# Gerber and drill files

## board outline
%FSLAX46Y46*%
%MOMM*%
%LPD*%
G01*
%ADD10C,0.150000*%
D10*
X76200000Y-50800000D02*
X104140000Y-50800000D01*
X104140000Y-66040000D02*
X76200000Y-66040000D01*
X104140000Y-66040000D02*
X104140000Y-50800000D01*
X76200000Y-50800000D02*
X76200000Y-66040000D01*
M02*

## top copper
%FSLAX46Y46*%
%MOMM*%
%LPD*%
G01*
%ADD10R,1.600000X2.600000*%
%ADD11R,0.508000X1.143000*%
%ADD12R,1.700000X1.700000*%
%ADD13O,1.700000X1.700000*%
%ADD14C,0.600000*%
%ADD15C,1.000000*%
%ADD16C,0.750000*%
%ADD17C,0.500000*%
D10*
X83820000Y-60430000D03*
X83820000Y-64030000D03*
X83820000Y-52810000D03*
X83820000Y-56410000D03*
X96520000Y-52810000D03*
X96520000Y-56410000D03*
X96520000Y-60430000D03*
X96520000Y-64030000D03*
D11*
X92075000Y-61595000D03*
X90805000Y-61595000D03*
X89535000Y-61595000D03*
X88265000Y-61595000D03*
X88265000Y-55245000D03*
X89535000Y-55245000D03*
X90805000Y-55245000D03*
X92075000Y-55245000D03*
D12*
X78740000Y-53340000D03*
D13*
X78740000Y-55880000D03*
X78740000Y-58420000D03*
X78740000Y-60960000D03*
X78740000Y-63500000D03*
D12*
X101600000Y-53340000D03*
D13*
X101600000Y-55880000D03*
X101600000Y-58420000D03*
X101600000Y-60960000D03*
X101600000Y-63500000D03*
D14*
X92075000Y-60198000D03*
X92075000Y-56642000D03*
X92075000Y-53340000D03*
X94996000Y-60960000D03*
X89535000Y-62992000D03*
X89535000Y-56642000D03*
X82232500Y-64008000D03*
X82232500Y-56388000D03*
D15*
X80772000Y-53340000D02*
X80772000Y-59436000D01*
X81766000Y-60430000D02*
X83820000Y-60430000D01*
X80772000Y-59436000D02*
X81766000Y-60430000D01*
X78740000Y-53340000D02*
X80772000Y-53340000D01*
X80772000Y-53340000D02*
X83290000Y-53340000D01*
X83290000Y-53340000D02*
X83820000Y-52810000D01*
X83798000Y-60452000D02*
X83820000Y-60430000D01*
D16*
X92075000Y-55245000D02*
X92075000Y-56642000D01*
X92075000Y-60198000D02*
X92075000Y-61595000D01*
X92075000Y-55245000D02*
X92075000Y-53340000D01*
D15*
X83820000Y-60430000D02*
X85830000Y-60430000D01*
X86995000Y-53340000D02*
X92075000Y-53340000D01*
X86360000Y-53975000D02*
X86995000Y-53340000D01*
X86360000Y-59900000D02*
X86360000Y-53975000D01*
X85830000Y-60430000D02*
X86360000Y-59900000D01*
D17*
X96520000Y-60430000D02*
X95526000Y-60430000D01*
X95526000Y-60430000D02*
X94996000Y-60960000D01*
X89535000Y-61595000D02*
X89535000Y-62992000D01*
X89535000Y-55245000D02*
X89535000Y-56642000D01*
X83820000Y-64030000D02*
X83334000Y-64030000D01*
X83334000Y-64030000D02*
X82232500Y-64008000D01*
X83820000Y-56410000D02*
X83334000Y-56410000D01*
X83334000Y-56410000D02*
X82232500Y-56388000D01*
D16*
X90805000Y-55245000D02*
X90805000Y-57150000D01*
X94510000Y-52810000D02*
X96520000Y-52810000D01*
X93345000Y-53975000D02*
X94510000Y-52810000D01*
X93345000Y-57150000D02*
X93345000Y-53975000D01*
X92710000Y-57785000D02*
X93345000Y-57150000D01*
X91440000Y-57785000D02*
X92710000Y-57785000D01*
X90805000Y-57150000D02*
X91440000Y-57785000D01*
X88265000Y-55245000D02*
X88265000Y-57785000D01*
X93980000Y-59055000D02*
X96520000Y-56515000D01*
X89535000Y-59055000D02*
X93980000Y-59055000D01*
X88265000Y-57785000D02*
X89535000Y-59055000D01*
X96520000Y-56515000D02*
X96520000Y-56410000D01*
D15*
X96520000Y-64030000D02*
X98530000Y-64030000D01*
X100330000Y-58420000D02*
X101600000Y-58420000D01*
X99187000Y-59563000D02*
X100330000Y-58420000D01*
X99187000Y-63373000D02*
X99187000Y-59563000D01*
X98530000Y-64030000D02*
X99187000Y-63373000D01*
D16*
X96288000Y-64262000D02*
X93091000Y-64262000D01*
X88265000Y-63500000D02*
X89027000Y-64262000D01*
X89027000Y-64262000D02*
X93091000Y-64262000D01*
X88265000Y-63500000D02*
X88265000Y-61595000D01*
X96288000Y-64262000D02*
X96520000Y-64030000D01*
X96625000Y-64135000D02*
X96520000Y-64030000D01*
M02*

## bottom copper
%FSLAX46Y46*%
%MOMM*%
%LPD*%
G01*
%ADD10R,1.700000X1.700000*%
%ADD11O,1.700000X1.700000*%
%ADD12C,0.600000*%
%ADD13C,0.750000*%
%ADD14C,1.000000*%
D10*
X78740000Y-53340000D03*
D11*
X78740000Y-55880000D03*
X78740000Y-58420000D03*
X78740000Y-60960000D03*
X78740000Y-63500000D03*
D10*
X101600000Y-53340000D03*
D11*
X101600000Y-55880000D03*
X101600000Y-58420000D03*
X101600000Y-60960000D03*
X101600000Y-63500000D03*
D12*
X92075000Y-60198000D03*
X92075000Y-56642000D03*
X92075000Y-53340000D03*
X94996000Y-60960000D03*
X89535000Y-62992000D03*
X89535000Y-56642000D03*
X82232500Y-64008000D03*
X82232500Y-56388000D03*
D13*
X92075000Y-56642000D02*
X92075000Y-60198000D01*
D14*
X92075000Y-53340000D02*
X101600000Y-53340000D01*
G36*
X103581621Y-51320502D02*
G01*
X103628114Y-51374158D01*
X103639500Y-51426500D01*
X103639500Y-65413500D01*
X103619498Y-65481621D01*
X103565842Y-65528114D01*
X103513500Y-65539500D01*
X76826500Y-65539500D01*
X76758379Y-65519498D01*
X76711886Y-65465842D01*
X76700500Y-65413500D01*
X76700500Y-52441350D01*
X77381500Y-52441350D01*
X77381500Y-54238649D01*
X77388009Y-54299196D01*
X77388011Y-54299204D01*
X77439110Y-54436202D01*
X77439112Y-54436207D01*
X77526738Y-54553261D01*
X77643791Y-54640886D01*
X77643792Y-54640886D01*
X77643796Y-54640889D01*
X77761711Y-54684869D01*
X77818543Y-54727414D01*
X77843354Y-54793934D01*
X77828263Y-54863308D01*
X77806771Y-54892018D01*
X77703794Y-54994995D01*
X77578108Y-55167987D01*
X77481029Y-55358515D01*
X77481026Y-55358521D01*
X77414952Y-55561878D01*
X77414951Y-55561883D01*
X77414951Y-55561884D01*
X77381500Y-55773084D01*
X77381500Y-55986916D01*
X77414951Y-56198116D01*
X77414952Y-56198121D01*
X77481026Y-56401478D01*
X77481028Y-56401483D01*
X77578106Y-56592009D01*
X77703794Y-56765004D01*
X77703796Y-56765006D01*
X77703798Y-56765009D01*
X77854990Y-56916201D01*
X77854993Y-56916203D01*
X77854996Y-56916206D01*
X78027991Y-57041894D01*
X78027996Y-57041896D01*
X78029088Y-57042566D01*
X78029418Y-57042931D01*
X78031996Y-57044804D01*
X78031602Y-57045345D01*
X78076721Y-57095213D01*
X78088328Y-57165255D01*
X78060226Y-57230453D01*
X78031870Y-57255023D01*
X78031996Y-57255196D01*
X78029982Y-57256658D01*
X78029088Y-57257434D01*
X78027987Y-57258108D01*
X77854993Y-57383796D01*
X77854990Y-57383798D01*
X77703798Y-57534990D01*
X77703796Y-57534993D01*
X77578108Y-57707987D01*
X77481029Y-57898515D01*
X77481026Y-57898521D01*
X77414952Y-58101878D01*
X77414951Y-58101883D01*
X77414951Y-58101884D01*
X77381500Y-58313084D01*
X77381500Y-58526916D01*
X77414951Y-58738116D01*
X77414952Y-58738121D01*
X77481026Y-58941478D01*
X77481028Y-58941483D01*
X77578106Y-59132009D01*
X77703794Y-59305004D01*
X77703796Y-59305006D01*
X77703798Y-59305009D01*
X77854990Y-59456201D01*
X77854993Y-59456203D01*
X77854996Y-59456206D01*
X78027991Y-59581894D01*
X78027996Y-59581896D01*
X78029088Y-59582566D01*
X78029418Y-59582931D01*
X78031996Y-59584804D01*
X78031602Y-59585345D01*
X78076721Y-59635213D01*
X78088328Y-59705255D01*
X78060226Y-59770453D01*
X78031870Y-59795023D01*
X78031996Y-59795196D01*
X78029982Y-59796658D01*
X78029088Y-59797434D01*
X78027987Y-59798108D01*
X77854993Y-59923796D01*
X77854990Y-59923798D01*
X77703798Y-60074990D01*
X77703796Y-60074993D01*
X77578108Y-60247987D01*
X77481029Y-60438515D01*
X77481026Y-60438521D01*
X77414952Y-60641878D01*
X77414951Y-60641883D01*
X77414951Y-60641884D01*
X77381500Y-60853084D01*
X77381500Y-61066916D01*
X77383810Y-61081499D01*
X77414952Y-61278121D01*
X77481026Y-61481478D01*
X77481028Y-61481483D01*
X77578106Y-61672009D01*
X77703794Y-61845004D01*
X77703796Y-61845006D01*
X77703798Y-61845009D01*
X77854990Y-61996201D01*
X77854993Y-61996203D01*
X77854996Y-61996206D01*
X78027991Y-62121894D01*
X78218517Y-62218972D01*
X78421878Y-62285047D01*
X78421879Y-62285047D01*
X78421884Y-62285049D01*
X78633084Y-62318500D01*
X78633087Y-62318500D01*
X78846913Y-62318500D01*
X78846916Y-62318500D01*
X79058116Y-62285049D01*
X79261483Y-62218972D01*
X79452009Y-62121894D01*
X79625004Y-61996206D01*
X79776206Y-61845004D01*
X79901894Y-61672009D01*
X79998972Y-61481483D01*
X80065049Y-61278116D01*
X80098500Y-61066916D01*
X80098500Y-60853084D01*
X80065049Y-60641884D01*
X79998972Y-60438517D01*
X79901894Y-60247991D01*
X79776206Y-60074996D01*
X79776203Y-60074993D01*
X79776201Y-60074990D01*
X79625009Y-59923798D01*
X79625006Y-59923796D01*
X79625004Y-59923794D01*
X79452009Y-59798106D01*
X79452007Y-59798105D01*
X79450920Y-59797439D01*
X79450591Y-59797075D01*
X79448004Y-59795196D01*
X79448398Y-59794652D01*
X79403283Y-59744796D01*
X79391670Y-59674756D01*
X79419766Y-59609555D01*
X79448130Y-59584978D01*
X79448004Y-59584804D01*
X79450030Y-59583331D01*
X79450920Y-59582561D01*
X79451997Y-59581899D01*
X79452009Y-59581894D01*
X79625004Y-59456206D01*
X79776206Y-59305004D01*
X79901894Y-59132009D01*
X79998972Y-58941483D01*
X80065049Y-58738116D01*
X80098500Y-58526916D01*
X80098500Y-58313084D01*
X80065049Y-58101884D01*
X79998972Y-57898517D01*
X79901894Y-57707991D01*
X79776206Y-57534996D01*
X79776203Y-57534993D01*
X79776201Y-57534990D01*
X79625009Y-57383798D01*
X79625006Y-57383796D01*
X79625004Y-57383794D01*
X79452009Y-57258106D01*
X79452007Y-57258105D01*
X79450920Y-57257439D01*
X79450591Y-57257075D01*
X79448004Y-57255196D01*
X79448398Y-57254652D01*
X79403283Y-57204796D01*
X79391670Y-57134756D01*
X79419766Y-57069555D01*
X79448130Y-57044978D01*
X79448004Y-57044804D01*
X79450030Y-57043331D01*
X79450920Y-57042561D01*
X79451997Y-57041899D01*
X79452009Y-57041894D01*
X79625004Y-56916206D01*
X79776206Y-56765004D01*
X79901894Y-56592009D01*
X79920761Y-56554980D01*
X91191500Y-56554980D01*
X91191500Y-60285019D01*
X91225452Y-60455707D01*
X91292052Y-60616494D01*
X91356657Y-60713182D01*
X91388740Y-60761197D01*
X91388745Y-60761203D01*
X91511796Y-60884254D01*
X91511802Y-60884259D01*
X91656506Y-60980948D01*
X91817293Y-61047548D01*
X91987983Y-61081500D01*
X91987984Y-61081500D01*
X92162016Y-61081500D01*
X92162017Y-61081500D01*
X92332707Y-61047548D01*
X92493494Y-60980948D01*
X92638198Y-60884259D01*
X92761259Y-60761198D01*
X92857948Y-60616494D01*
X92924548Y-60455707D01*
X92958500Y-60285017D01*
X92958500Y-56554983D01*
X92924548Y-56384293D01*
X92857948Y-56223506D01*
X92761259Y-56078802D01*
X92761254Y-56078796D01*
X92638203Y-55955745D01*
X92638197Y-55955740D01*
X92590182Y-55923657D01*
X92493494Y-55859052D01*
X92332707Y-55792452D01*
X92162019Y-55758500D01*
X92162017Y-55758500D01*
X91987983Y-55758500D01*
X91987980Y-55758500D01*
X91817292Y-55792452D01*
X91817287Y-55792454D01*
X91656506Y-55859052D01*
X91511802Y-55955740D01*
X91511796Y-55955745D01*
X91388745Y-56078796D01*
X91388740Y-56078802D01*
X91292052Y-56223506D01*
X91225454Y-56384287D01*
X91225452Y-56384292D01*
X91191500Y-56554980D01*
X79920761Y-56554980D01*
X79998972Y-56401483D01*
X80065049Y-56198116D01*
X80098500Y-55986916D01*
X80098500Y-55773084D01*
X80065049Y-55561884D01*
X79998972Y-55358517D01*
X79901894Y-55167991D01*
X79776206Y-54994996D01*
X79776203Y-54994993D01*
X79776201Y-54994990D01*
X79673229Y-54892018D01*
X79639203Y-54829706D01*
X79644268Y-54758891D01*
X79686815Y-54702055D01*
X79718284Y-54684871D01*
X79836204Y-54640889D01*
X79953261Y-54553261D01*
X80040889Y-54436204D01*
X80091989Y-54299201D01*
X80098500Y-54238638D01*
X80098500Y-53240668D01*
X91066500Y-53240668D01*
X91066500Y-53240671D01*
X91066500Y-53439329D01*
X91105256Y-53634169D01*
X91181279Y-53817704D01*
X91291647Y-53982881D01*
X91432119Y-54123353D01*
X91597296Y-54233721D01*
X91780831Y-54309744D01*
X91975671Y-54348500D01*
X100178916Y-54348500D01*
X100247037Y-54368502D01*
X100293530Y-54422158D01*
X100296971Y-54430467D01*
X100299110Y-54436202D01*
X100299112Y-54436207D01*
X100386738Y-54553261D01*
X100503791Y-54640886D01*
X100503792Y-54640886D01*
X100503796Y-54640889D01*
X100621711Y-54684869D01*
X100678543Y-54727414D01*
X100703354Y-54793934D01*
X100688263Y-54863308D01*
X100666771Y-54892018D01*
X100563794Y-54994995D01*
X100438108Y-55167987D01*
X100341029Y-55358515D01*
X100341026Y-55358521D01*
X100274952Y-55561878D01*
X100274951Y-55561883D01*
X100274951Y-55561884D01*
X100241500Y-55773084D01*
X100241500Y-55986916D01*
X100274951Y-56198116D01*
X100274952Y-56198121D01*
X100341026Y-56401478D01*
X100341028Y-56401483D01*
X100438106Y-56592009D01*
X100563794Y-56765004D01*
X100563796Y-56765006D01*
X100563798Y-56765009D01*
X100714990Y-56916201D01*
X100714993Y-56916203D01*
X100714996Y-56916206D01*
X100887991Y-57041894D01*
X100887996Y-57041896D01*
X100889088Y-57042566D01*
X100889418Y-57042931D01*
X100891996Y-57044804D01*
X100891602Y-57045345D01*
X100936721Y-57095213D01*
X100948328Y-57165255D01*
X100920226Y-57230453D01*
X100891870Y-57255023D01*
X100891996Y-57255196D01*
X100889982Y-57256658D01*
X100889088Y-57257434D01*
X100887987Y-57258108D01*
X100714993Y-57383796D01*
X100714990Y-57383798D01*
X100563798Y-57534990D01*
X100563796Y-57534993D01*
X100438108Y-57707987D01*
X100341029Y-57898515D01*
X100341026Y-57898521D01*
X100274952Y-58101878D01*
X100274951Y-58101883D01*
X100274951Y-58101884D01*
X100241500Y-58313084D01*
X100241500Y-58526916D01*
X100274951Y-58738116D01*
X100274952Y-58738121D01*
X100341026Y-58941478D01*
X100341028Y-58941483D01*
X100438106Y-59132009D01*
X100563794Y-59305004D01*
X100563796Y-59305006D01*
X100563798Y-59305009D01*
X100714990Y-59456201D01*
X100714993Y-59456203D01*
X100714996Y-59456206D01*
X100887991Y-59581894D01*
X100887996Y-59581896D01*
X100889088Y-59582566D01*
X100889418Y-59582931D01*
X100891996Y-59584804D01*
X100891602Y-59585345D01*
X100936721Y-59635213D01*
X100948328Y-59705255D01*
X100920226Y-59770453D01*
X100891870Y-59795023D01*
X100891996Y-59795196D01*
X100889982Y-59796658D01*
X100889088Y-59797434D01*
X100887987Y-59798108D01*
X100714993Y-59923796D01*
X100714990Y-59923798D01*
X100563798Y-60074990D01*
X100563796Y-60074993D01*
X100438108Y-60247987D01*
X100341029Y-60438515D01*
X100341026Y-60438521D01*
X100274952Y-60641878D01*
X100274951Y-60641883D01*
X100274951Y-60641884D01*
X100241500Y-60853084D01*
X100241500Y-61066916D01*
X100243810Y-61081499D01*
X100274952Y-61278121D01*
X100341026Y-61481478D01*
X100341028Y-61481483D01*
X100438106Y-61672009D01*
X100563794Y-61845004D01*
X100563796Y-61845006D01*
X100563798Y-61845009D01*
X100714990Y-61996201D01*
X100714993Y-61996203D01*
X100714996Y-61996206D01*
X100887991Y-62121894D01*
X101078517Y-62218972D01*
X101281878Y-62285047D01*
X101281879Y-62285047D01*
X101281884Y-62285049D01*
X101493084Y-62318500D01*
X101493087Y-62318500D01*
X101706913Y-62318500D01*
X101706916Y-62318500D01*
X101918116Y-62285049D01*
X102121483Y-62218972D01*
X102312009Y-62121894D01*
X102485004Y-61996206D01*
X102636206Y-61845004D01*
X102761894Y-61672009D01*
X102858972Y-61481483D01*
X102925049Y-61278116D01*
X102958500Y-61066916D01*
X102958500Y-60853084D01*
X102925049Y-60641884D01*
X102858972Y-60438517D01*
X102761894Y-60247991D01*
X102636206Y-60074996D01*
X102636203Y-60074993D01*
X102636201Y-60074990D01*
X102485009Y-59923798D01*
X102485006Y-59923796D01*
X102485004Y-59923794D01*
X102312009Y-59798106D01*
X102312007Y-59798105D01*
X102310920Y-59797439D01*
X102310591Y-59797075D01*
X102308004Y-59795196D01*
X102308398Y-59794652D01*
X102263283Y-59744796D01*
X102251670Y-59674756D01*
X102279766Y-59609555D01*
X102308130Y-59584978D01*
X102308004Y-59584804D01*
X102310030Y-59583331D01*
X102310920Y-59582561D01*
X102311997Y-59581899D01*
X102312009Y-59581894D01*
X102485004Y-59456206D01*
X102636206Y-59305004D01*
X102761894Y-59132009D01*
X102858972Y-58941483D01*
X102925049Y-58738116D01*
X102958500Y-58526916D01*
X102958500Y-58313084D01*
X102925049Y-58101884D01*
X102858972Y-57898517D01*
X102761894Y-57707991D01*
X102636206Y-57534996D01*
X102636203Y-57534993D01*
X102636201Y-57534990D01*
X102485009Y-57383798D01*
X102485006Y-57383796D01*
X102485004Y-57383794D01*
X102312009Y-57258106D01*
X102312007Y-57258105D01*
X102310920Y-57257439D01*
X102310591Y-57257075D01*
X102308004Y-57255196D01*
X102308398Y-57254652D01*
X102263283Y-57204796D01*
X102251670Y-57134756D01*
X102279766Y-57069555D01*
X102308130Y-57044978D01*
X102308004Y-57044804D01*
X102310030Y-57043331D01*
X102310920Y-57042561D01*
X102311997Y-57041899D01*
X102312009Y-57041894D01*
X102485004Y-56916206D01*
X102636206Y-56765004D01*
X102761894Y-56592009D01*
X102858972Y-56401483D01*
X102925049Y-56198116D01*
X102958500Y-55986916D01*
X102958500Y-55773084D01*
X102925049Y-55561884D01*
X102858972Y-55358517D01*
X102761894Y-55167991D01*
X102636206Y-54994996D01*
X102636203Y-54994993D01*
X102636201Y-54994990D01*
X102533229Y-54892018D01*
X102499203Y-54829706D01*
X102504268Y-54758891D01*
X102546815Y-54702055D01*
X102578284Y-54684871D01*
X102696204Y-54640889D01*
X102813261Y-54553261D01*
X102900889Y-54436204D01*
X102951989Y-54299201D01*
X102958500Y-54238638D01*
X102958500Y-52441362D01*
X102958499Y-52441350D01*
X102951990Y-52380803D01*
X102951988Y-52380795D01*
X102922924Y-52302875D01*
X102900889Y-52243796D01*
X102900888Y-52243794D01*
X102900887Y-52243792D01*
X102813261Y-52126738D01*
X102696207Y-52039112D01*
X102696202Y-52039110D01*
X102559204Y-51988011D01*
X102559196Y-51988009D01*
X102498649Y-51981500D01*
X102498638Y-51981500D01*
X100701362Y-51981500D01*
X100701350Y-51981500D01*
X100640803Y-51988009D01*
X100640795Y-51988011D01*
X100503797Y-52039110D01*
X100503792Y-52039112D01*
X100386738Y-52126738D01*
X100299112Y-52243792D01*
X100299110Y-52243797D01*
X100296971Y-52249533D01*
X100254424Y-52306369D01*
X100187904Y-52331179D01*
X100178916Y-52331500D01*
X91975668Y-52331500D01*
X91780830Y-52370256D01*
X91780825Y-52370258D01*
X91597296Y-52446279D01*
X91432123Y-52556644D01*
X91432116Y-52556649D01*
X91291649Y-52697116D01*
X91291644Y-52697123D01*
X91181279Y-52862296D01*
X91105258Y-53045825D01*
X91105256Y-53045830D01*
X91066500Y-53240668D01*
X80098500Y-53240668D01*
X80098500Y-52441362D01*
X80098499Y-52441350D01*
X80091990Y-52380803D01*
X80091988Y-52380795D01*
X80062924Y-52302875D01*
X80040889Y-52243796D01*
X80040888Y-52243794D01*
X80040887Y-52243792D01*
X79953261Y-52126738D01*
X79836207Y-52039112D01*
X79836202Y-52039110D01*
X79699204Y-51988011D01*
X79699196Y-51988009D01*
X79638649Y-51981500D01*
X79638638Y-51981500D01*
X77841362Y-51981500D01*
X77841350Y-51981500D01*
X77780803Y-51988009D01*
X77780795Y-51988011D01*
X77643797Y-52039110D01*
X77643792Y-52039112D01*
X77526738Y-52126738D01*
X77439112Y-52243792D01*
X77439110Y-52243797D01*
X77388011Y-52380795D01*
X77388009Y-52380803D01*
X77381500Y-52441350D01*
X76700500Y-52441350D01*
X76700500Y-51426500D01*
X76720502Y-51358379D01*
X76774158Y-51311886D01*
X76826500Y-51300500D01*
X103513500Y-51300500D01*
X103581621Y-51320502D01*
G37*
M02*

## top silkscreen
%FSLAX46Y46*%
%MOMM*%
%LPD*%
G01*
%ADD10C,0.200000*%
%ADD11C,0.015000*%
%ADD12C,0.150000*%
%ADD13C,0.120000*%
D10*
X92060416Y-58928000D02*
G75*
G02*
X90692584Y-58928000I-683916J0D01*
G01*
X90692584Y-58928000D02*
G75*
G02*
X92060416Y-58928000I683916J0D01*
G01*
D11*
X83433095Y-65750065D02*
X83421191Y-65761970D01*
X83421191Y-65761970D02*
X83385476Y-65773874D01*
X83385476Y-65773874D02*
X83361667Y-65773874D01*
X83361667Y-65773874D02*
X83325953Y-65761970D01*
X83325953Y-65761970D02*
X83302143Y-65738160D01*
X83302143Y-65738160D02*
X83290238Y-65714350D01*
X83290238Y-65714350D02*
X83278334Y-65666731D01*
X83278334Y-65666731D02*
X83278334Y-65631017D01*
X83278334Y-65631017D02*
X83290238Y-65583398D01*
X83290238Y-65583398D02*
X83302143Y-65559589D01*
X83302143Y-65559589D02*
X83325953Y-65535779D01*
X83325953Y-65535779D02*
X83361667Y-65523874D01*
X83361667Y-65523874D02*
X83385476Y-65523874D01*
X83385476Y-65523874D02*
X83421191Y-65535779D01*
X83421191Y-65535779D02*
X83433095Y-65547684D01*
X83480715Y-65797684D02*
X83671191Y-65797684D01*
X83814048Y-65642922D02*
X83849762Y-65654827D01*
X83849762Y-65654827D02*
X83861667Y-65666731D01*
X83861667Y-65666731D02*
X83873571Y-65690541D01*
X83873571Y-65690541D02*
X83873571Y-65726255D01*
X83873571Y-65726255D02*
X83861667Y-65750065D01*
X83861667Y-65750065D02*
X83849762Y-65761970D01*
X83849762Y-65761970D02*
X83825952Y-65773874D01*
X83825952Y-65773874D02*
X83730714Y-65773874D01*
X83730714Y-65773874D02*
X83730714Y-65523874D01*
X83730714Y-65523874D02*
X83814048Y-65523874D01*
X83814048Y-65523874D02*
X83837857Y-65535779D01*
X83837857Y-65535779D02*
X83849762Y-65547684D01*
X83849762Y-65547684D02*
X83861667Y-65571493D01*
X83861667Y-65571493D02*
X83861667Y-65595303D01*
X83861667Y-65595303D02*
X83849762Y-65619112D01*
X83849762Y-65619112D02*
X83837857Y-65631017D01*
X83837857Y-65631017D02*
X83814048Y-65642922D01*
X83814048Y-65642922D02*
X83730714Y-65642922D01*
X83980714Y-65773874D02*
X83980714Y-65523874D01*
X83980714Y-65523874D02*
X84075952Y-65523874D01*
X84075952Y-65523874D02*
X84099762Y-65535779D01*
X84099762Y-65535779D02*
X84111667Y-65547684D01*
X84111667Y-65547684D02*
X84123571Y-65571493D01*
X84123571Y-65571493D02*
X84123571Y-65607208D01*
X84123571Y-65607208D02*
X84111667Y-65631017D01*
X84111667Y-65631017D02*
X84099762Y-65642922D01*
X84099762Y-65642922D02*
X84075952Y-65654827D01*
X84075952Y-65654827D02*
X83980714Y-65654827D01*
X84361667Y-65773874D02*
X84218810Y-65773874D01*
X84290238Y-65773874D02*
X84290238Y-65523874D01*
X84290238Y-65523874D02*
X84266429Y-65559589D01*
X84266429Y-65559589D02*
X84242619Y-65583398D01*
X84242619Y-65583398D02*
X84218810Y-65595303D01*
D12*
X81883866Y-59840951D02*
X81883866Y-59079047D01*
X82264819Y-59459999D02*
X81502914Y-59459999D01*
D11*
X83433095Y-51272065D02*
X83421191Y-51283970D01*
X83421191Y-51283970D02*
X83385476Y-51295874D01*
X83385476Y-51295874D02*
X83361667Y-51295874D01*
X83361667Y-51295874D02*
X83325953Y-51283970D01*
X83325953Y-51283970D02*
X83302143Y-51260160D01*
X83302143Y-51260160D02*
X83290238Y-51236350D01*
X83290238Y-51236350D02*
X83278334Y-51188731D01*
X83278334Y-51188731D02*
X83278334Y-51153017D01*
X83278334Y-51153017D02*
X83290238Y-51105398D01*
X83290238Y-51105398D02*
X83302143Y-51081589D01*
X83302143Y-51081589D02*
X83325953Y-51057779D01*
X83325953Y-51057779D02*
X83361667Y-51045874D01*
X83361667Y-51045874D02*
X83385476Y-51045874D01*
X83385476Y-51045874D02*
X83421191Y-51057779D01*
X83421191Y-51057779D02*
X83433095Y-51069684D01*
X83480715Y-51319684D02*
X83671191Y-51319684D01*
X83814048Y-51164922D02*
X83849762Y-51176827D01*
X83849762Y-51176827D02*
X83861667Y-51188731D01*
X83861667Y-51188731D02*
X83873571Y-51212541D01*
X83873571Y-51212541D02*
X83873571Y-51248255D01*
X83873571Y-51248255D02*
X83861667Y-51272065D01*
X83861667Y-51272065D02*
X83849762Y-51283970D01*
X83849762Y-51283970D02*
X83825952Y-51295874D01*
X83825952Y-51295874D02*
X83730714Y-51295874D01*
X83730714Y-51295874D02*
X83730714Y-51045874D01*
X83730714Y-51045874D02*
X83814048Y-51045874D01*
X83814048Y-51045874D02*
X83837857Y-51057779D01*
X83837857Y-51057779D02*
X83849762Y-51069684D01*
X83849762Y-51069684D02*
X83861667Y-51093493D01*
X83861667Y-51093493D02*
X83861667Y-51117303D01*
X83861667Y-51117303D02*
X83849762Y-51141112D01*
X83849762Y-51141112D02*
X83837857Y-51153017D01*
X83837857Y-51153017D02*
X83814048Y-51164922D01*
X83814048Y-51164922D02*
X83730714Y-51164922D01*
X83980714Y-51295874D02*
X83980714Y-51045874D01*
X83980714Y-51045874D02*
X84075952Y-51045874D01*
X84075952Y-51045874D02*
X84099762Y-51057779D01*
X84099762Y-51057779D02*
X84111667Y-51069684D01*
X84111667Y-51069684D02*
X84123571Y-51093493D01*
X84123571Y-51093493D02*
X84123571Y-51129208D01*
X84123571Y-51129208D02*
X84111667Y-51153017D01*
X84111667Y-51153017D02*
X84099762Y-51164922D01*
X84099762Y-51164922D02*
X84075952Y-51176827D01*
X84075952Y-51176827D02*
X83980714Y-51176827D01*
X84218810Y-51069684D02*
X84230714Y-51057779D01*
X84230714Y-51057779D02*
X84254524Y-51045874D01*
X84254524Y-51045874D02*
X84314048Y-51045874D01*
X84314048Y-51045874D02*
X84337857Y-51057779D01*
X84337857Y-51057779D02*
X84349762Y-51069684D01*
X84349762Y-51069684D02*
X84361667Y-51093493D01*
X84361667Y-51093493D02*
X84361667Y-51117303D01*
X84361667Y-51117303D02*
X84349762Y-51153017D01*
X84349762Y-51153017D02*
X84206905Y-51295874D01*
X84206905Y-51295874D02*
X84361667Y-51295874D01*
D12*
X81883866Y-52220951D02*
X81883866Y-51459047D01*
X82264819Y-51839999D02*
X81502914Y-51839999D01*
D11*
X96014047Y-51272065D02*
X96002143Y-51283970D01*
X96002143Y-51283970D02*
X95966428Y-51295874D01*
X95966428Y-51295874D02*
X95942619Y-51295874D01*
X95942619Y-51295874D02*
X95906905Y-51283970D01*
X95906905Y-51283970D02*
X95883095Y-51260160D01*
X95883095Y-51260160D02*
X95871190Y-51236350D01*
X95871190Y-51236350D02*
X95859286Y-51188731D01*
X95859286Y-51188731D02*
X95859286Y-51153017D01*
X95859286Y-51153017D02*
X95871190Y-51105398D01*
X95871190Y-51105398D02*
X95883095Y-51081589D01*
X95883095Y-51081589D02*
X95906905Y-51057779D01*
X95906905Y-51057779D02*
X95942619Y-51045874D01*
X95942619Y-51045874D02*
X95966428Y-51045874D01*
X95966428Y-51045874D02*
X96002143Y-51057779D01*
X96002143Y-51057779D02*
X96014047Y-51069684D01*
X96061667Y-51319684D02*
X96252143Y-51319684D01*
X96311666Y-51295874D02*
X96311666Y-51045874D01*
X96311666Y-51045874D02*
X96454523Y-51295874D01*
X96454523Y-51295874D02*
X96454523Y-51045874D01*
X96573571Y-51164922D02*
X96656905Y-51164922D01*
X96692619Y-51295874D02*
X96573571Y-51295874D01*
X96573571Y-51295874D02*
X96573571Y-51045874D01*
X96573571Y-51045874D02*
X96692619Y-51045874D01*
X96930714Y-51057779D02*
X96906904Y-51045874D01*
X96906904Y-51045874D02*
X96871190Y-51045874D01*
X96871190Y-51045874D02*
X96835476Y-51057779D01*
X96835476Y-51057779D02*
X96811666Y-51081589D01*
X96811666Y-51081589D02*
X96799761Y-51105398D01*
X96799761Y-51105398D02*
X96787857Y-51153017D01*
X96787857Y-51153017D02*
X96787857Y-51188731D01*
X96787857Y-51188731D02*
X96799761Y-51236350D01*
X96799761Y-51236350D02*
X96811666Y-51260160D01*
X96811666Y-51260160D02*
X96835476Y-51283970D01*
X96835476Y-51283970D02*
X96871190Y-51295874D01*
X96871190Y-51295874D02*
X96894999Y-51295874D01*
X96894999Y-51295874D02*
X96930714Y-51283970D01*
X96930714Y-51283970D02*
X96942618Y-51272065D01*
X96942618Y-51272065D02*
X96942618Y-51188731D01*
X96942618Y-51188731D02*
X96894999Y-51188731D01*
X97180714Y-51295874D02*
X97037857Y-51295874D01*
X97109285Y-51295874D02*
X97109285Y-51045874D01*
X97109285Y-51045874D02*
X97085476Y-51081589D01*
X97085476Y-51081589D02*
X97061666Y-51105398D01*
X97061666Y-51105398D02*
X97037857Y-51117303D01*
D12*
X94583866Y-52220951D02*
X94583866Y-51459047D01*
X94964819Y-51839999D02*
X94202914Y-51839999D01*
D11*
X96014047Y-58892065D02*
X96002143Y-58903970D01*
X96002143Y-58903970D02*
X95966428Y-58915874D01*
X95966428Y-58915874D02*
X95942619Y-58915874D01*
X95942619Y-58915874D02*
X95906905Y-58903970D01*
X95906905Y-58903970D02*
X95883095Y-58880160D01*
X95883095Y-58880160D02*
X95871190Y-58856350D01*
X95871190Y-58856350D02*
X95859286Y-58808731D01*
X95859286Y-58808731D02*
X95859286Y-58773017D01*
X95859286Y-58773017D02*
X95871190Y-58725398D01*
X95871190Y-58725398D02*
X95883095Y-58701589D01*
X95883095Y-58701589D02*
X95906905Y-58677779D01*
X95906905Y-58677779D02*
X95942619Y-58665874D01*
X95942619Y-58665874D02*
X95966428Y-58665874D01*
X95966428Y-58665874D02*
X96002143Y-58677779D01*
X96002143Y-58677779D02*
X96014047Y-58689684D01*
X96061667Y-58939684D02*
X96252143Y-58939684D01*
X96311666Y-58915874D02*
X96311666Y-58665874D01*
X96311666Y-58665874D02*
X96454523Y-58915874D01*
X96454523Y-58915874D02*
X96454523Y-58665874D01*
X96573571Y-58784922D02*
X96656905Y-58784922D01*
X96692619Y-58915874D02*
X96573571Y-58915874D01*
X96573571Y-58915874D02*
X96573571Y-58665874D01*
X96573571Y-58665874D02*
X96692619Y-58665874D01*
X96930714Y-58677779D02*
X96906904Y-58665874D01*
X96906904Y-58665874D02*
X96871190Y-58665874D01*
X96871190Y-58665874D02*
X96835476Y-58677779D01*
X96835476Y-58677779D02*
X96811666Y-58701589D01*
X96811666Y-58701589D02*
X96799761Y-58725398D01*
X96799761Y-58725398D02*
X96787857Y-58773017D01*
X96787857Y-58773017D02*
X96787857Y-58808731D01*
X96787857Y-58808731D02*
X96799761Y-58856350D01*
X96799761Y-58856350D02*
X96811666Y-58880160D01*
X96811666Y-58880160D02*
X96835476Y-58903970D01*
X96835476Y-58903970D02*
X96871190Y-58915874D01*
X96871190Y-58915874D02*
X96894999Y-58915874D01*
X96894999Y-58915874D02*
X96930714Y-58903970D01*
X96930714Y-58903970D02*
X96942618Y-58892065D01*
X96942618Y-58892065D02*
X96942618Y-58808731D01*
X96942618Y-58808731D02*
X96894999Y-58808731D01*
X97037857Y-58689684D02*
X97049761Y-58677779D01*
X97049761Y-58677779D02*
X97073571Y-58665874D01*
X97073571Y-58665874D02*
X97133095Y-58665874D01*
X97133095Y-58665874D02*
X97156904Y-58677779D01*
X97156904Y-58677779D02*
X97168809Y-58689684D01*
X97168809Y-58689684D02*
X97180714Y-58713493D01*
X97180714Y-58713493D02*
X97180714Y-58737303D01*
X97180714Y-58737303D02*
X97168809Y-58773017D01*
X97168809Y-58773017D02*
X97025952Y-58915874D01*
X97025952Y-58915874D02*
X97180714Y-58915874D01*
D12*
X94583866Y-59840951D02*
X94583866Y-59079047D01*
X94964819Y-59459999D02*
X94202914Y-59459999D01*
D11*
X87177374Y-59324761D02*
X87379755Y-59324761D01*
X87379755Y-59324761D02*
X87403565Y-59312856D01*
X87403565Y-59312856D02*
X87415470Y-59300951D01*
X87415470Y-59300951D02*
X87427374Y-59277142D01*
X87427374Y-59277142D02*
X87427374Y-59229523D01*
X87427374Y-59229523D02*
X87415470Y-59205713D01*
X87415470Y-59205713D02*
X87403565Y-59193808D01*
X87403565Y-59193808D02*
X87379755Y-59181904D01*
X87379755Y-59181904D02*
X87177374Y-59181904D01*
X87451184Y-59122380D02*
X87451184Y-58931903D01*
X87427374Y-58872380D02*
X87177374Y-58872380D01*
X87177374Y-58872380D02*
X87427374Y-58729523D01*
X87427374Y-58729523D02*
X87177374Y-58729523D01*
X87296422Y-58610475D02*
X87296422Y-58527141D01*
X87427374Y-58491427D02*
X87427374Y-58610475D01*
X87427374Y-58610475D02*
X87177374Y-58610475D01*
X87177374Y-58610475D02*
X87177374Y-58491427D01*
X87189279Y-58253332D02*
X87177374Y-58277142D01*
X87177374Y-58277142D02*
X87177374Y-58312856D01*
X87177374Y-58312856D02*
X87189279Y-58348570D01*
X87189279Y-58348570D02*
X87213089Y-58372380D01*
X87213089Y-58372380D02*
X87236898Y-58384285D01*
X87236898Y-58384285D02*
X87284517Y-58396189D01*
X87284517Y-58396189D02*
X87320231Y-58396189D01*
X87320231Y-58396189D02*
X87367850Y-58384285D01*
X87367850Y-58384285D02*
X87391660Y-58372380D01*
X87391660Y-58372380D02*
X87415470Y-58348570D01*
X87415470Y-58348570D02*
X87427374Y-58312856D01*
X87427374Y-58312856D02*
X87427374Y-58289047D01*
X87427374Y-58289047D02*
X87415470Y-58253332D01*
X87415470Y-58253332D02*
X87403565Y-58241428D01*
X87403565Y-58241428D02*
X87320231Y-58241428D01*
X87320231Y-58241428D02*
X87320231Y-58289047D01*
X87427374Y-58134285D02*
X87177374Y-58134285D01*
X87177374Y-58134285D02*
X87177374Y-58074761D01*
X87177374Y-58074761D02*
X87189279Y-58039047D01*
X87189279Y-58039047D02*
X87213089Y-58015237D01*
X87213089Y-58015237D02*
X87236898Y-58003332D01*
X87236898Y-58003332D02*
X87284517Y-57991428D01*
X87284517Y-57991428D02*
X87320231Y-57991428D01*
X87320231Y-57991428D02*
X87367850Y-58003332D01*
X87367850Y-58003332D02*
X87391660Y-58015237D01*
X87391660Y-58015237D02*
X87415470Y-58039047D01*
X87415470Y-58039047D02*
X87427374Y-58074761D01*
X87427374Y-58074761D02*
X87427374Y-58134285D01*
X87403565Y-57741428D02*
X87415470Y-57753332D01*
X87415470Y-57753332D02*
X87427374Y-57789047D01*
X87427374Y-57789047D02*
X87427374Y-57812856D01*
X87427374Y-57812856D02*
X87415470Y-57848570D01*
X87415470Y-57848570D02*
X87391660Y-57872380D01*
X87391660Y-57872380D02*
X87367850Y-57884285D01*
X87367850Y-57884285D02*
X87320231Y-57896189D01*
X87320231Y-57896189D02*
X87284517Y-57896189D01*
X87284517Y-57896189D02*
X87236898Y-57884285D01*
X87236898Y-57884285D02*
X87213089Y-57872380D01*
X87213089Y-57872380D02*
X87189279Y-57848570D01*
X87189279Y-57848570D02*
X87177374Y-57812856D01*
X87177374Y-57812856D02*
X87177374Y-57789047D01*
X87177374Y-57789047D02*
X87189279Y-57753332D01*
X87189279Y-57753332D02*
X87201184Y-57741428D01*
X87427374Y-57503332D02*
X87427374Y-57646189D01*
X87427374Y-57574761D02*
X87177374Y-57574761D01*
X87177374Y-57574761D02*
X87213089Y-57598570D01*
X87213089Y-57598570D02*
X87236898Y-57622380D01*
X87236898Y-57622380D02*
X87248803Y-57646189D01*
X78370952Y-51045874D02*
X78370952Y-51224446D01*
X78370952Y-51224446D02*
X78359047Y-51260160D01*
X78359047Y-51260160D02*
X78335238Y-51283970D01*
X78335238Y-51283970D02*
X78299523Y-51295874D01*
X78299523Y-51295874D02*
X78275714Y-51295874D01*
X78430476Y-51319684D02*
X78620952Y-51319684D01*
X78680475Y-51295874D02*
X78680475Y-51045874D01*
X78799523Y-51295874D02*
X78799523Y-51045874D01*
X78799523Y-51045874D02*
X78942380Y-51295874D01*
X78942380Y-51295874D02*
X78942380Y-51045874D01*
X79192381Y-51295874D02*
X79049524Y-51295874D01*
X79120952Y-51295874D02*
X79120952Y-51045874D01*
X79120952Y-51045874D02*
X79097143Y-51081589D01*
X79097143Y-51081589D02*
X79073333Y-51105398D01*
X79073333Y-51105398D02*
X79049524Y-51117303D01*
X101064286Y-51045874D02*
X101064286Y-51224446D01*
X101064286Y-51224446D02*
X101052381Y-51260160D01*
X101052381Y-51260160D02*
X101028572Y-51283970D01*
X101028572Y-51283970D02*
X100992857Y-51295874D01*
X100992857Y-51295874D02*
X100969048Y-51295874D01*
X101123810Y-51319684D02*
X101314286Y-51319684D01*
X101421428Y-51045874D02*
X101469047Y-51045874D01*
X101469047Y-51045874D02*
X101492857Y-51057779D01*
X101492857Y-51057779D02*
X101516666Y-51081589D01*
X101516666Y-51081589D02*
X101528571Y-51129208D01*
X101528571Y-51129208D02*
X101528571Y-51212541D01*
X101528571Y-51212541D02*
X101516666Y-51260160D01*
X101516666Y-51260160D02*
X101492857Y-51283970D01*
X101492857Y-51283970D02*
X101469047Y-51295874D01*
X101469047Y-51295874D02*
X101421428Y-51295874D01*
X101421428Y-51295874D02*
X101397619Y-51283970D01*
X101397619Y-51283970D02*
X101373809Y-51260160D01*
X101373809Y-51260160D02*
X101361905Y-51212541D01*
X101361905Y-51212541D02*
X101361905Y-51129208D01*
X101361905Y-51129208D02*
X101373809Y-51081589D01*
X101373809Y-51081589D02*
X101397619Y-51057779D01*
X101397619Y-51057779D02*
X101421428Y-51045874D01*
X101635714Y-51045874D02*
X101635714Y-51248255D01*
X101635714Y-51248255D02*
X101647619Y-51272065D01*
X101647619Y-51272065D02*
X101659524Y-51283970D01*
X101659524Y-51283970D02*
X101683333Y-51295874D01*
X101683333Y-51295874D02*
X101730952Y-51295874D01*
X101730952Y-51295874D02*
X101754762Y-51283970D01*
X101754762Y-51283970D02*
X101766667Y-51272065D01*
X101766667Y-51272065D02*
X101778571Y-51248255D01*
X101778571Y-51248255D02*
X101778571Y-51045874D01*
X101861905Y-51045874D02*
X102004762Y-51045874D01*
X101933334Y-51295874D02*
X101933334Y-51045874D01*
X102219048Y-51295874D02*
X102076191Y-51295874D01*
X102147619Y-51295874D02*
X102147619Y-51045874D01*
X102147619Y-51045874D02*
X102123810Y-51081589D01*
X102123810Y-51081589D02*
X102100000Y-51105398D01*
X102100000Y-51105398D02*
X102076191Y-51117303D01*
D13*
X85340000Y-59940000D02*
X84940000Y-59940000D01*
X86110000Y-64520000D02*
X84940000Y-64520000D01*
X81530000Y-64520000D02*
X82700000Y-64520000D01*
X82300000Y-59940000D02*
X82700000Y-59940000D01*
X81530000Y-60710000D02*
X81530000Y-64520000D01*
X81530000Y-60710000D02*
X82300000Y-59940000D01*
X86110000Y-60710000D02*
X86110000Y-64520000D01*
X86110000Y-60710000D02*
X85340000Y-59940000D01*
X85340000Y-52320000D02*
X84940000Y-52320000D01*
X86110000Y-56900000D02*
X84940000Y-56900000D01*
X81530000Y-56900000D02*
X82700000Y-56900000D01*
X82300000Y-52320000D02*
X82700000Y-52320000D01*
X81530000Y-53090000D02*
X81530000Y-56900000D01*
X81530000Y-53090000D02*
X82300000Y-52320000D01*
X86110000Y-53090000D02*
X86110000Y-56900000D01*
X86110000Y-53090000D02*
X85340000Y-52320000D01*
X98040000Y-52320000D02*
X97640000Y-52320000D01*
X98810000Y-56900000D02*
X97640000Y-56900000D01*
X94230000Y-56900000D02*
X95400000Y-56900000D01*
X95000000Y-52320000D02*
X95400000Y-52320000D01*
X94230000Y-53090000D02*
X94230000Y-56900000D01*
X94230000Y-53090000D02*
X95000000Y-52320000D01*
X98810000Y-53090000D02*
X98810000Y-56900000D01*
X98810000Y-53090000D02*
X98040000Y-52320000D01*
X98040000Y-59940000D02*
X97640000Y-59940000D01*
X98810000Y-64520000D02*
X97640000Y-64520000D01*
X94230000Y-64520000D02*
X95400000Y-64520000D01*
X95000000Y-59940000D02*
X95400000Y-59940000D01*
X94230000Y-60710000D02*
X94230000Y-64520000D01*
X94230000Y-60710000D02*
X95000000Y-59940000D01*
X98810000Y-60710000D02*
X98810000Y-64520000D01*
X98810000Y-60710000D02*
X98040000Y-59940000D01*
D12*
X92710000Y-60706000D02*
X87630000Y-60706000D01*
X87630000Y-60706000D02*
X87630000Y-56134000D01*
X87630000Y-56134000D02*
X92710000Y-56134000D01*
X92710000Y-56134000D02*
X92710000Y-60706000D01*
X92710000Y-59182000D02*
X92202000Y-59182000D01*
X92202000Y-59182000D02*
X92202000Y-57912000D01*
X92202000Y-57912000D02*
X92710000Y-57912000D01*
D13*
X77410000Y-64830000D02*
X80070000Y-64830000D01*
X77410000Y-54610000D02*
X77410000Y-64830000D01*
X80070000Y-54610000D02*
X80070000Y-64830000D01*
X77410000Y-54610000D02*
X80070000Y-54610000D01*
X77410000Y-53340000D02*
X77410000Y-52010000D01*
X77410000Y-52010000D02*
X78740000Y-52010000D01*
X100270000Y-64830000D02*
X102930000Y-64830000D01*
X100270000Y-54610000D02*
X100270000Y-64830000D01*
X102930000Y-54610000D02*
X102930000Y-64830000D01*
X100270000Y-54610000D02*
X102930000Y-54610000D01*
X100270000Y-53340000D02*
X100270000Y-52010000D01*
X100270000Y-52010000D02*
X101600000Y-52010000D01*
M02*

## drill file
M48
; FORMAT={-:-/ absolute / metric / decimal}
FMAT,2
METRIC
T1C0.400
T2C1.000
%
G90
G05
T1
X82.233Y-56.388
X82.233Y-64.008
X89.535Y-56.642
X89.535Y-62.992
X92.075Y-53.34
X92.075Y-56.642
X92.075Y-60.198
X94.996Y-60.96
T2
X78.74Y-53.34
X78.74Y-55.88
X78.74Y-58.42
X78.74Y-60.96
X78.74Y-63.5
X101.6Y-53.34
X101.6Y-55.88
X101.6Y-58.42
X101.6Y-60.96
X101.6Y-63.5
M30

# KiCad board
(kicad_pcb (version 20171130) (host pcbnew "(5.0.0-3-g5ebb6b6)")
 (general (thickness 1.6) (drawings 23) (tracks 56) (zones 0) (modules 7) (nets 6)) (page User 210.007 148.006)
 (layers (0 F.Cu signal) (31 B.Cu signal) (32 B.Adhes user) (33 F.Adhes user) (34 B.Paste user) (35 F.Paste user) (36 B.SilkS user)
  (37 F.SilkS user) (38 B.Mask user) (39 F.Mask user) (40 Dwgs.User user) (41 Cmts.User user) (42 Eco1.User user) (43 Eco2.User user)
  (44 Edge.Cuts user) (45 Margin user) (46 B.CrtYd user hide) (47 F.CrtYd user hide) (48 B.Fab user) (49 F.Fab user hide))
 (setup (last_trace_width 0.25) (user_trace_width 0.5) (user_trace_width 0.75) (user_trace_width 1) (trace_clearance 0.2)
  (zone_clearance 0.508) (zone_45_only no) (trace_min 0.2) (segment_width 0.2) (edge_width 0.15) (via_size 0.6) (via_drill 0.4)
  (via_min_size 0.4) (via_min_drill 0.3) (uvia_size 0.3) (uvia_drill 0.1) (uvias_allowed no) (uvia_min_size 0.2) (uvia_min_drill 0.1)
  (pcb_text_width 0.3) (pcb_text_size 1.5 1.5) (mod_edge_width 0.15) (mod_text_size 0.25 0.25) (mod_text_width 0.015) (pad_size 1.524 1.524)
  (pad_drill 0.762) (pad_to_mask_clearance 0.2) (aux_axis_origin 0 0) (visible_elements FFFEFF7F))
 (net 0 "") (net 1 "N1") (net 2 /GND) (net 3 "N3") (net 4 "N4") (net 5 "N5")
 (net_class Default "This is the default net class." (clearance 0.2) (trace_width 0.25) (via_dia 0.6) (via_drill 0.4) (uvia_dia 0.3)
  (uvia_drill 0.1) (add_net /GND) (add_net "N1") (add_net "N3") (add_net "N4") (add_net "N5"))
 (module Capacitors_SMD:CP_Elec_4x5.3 (layer F.Cu) (at 83.82 62.23 270)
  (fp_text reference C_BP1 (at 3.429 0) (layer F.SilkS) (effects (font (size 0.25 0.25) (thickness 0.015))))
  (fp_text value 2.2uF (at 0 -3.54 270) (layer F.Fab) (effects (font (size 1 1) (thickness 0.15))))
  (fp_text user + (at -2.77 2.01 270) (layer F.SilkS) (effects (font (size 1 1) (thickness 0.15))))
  (fp_line (start -2.29 -1.52) (end -2.29 -1.12) (layer F.SilkS) (width 0.12))
  (fp_line (start 2.29 -2.29) (end 2.29 -1.12) (layer F.SilkS) (width 0.12))
  (fp_line (start 2.29 2.29) (end 2.29 1.12) (layer F.SilkS) (width 0.12))
  (fp_line (start -2.29 1.52) (end -2.29 1.12) (layer F.SilkS) (width 0.12))
  (fp_line (start -1.52 2.29) (end 2.29 2.29) (layer F.SilkS) (width 0.12))
  (fp_line (start -1.52 2.29) (end -2.29 1.52) (layer F.SilkS) (width 0.12))
  (fp_line (start -1.52 -2.29) (end 2.29 -2.29) (layer F.SilkS) (width 0.12))
  (fp_line (start -1.52 -2.29) (end -2.29 -1.52) (layer F.SilkS) (width 0.12))
  (pad 1 smd rect (at -1.8 0 90) (size 2.6 1.6) (layers F.Cu F.Paste F.Mask) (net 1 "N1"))
  (pad 2 smd rect (at 1.8 0 90) (size 2.6 1.6) (layers F.Cu F.Paste F.Mask) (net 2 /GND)))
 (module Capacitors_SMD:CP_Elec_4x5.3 (layer F.Cu) (at 83.82 54.61 270)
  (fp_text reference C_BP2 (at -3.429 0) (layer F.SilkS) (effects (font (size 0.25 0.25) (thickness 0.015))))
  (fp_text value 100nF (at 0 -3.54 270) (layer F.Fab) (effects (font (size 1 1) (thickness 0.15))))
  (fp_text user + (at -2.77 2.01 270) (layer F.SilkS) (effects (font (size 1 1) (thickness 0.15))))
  (fp_line (start -2.29 -1.52) (end -2.29 -1.12) (layer F.SilkS) (width 0.12))
  (fp_line (start 2.29 -2.29) (end 2.29 -1.12) (layer F.SilkS) (width 0.12))
  (fp_line (start 2.29 2.29) (end 2.29 1.12) (layer F.SilkS) (width 0.12))
  (fp_line (start -2.29 1.52) (end -2.29 1.12) (layer F.SilkS) (width 0.12))
  (fp_line (start -1.52 2.29) (end 2.29 2.29) (layer F.SilkS) (width 0.12))
  (fp_line (start -1.52 2.29) (end -2.29 1.52) (layer F.SilkS) (width 0.12))
  (fp_line (start -1.52 -2.29) (end 2.29 -2.29) (layer F.SilkS) (width 0.12))
  (fp_line (start -1.52 -2.29) (end -2.29 -1.52) (layer F.SilkS) (width 0.12))
  (pad 1 smd rect (at -1.8 0 90) (size 2.6 1.6) (layers F.Cu F.Paste F.Mask) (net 1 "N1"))
  (pad 2 smd rect (at 1.8 0 90) (size 2.6 1.6) (layers F.Cu F.Paste F.Mask) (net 2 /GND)))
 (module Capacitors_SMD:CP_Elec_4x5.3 (layer F.Cu) (at 96.52 54.61 270)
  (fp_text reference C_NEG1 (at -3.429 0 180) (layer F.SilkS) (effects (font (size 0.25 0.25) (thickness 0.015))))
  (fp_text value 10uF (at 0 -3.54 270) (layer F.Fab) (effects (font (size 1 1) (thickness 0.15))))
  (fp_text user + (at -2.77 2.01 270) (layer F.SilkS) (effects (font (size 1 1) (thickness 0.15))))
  (fp_line (start -2.29 -1.52) (end -2.29 -1.12) (layer F.SilkS) (width 0.12))
  (fp_line (start 2.29 -2.29) (end 2.29 -1.12) (layer F.SilkS) (width 0.12))
  (fp_line (start 2.29 2.29) (end 2.29 1.12) (layer F.SilkS) (width 0.12))
  (fp_line (start -2.29 1.52) (end -2.29 1.12) (layer F.SilkS) (width 0.12))
  (fp_line (start -1.52 2.29) (end 2.29 2.29) (layer F.SilkS) (width 0.12))
  (fp_line (start -1.52 2.29) (end -2.29 1.52) (layer F.SilkS) (width 0.12))
  (fp_line (start -1.52 -2.29) (end 2.29 -2.29) (layer F.SilkS) (width 0.12))
  (fp_line (start -1.52 -2.29) (end -2.29 -1.52) (layer F.SilkS) (width 0.12))
  (pad 1 smd rect (at -1.8 0 90) (size 2.6 1.6) (layers F.Cu F.Paste F.Mask) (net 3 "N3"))
  (pad 2 smd rect (at 1.8 0 90) (size 2.6 1.6) (layers F.Cu F.Paste F.Mask) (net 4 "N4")))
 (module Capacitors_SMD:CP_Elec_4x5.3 (layer F.Cu) (at 96.52 62.23 270)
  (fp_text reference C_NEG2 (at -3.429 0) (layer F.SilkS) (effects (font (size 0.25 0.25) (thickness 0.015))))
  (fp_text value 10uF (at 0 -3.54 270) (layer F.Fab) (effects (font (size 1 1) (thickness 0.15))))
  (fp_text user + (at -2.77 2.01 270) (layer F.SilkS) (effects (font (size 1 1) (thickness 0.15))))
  (fp_line (start -2.29 -1.52) (end -2.29 -1.12) (layer F.SilkS) (width 0.12))
  (fp_line (start 2.29 -2.29) (end 2.29 -1.12) (layer F.SilkS) (width 0.12))
  (fp_line (start 2.29 2.29) (end 2.29 1.12) (layer F.SilkS) (width 0.12))
  (fp_line (start -2.29 1.52) (end -2.29 1.12) (layer F.SilkS) (width 0.12))
  (fp_line (start -1.52 2.29) (end 2.29 2.29) (layer F.SilkS) (width 0.12))
  (fp_line (start -1.52 2.29) (end -2.29 1.52) (layer F.SilkS) (width 0.12))
  (fp_line (start -1.52 -2.29) (end 2.29 -2.29) (layer F.SilkS) (width 0.12))
  (fp_line (start -1.52 -2.29) (end -2.29 -1.52) (layer F.SilkS) (width 0.12))
  (pad 1 smd rect (at -1.8 0 90) (size 2.6 1.6) (layers F.Cu F.Paste F.Mask) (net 2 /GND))
  (pad 2 smd rect (at 1.8 0 90) (size 2.6 1.6) (layers F.Cu F.Paste F.Mask) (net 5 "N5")))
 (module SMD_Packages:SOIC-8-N (layer F.Cu) (at 90.17 58.42 180)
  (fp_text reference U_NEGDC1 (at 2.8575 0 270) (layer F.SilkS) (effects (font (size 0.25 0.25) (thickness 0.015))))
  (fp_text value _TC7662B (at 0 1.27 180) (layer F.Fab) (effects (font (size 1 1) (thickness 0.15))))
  (fp_line (start -2.54 -2.286) (end 2.54 -2.286) (layer F.SilkS) (width 0.15))
  (fp_line (start 2.54 -2.286) (end 2.54 2.286) (layer F.SilkS) (width 0.15))
  (fp_line (start 2.54 2.286) (end -2.54 2.286) (layer F.SilkS) (width 0.15))
  (fp_line (start -2.54 2.286) (end -2.54 -2.286) (layer F.SilkS) (width 0.15))
  (fp_line (start -2.54 -0.762) (end -2.032 -0.762) (layer F.SilkS) (width 0.15))
  (fp_line (start -2.032 -0.762) (end -2.032 0.508) (layer F.SilkS) (width 0.15))
  (fp_line (start -2.032 0.508) (end -2.54 0.508) (layer F.SilkS) (width 0.15))
  (pad 8 smd rect (at -1.905 -3.175 180) (size 0.508 1.143) (layers F.Cu F.Paste F.Mask) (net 1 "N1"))
  (pad 7 smd rect (at -0.635 -3.175 180) (size 0.508 1.143) (layers F.Cu F.Paste F.Mask))
  (pad 6 smd rect (at 0.635 -3.175 180) (size 0.508 1.143) (layers F.Cu F.Paste F.Mask) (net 2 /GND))
  (pad 5 smd rect (at 1.905 -3.175 180) (size 0.508 1.143) (layers F.Cu F.Paste F.Mask) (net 5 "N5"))
  (pad 4 smd rect (at 1.905 3.175 180) (size 0.508 1.143) (layers F.Cu F.Paste F.Mask) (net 4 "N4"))
  (pad 3 smd rect (at 0.635 3.175 180) (size 0.508 1.143) (layers F.Cu F.Paste F.Mask) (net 2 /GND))
  (pad 2 smd rect (at -0.635 3.175 180) (size 0.508 1.143) (layers F.Cu F.Paste F.Mask) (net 3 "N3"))
  (pad 1 smd rect (at -1.905 3.175 180) (size 0.508 1.143) (layers F.Cu F.Paste F.Mask) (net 1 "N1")))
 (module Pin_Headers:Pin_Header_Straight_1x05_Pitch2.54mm (layer F.Cu) (at 78.74 53.34)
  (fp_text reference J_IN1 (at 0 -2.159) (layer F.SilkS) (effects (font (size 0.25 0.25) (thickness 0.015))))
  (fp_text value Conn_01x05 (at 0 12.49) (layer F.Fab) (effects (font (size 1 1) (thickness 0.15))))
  (fp_line (start -1.33 11.49) (end 1.33 11.49) (layer F.SilkS) (width 0.12))
  (fp_line (start -1.33 1.27) (end -1.33 11.49) (layer F.SilkS) (width 0.12))
  (fp_line (start 1.33 1.27) (end 1.33 11.49) (layer F.SilkS) (width 0.12))
  (fp_line (start -1.33 1.27) (end 1.33 1.27) (layer F.SilkS) (width 0.12))
  (fp_line (start -1.33 0) (end -1.33 -1.33) (layer F.SilkS) (width 0.12))
  (fp_line (start -1.33 -1.33) (end 0 -1.33) (layer F.SilkS) (width 0.12))
  (pad 1 thru_hole rect (at 0 0) (size 1.7 1.7) (drill 1) (layers *.Cu *.Mask) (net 1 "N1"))
  (pad 2 thru_hole oval (at 0 2.54) (size 1.7 1.7) (drill 1) (layers *.Cu *.Mask))
  (pad 3 thru_hole oval (at 0 5.08) (size 1.7 1.7) (drill 1) (layers *.Cu *.Mask))
  (pad 4 thru_hole oval (at 0 7.62) (size 1.7 1.7) (drill 1) (layers *.Cu *.Mask))
  (pad 5 thru_hole oval (at 0 10.16) (size 1.7 1.7) (drill 1) (layers *.Cu *.Mask) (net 2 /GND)))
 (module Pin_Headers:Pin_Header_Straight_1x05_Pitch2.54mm (layer F.Cu) (at 101.6 53.34)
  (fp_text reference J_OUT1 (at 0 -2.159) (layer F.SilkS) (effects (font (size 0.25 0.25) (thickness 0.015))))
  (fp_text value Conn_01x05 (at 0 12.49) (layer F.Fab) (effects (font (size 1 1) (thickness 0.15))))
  (fp_line (start -1.33 11.49) (end 1.33 11.49) (layer F.SilkS) (width 0.12))
  (fp_line (start -1.33 1.27) (end -1.33 11.49) (layer F.SilkS) (width 0.12))
  (fp_line (start 1.33 1.27) (end 1.33 11.49) (layer F.SilkS) (width 0.12))
  (fp_line (start -1.33 1.27) (end 1.33 1.27) (layer F.SilkS) (width 0.12))
  (fp_line (start -1.33 0) (end -1.33 -1.33) (layer F.SilkS) (width 0.12))
  (fp_line (start -1.33 -1.33) (end 0 -1.33) (layer F.SilkS) (width 0.12))
  (pad 1 thru_hole rect (at 0 0) (size 1.7 1.7) (drill 1) (layers *.Cu *.Mask) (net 1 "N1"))
  (pad 2 thru_hole oval (at 0 2.54) (size 1.7 1.7) (drill 1) (layers *.Cu *.Mask))
  (pad 3 thru_hole oval (at 0 5.08) (size 1.7 1.7) (drill 1) (layers *.Cu *.Mask) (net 5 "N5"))
  (pad 4 thru_hole oval (at 0 7.62) (size 1.7 1.7) (drill 1) (layers *.Cu *.Mask))
  (pad 5 thru_hole oval (at 0 10.16) (size 1.7 1.7) (drill 1) (layers *.Cu *.Mask) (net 2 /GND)))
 (gr_line (start 76.2 50.8) (end 104.14 50.8) (angle 90) (layer Edge.Cuts) (width 0.15))
 (gr_line (start 104.14 66.04) (end 76.2 66.04) (angle 90) (layer Edge.Cuts) (width 0.15))
 (gr_line (start 104.14 66.04) (end 104.14 50.8) (angle 90) (layer Edge.Cuts) (width 0.15))
 (gr_circle (center 91.3765 58.928) (end 91.6305 59.563) (layer F.SilkS) (width 0.2))
 (gr_line (start 76.2 50.8) (end 76.2 66.04) (angle 90) (layer Edge.Cuts) (width 0.15))
 (segment (start 80.772 53.34) (end 80.772 59.436) (width 1) (layer F.Cu) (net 1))
 (segment (start 81.766 60.43) (end 83.82 60.43) (width 1) (layer F.Cu) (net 1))
 (segment (start 80.772 59.436) (end 81.766 60.43) (width 1) (layer F.Cu) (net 1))
 (segment (start 78.74 53.34) (end 80.772 53.34) (width 1) (layer F.Cu) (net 1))
 (segment (start 80.772 53.34) (end 83.29 53.34) (width 1) (layer F.Cu) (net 1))
 (segment (start 83.29 53.34) (end 83.82 52.81) (width 1) (layer F.Cu) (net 1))
 (segment (start 83.798 60.452) (end 83.82 60.43) (width 1) (layer F.Cu) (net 1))
 (segment (start 92.075 55.245) (end 92.075 56.642) (width 0.75) (layer F.Cu) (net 1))
 (segment (start 92.075 60.198) (end 92.075 61.595) (width 0.75) (layer F.Cu) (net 1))
 (via (at 92.075 60.198) (size 0.6) (drill 0.4) (layers F.Cu B.Cu) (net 1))
 (segment (start 92.075 56.642) (end 92.075 60.198) (width 0.75) (layer B.Cu) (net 1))
 (via (at 92.075 56.642) (size 0.6) (drill 0.4) (layers F.Cu B.Cu) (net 1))
 (segment (start 92.075 55.245) (end 92.075 53.34) (width 0.75) (layer F.Cu) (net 1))
 (segment (start 83.82 60.43) (end 85.83 60.43) (width 1) (layer F.Cu) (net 1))
 (segment (start 86.995 53.34) (end 92.075 53.34) (width 1) (layer F.Cu) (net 1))
 (segment (start 86.36 53.975) (end 86.995 53.34) (width 1) (layer F.Cu) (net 1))
 (segment (start 86.36 59.9) (end 86.36 53.975) (width 1) (layer F.Cu) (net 1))
 (segment (start 85.83 60.43) (end 86.36 59.9) (width 1) (layer F.Cu) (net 1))
 (segment (start 92.075 53.34) (end 101.6 53.34) (width 1) (layer B.Cu) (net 1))
 (via (at 92.075 53.34) (size 0.6) (drill 0.4) (layers F.Cu B.Cu) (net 1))
 (segment (start 96.52 60.43) (end 95.526 60.43) (width 0.5) (layer F.Cu) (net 2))
 (via (at 94.996 60.96) (size 0.6) (drill 0.4) (layers F.Cu B.Cu) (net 2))
 (segment (start 95.526 60.43) (end 94.996 60.96) (width 0.5) (layer F.Cu) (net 2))
 (segment (start 89.535 61.595) (end 89.535 62.992) (width 0.5) (layer F.Cu) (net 2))
 (via (at 89.535 62.992) (size 0.6) (drill 0.4) (layers F.Cu B.Cu) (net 2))
 (segment (start 89.535 55.245) (end 89.535 56.642) (width 0.5) (layer F.Cu) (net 2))
 (via (at 89.535 56.642) (size 0.6) (drill 0.4) (layers F.Cu B.Cu) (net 2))
 (segment (start 83.82 64.03) (end 83.334 64.03) (width 0.5) (layer F.Cu) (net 2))
 (segment (start 83.334 64.03) (end 82.2325 64.008) (width 0.5) (layer F.Cu) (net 2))
 (via (at 82.2325 64.008) (size 0.6) (drill 0.4) (layers F.Cu B.Cu) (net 2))
 (segment (start 83.82 56.41) (end 83.334 56.41) (width 0.5) (layer F.Cu) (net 2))
 (segment (start 83.334 56.41) (end 82.2325 56.388) (width 0.5) (layer F.Cu) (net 2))
 (via (at 82.2325 56.388) (size 0.6) (drill 0.4) (layers F.Cu B.Cu) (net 2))
 (segment (start 90.805 55.245) (end 90.805 57.15) (width 0.75) (layer F.Cu) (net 3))
 (segment (start 94.51 52.81) (end 96.52 52.81) (width 0.75) (layer F.Cu) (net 3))
 (segment (start 93.345 53.975) (end 94.51 52.81) (width 0.75) (layer F.Cu) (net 3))
 (segment (start 93.345 57.15) (end 93.345 53.975) (width 0.75) (layer F.Cu) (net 3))
 (segment (start 92.71 57.785) (end 93.345 57.15) (width 0.75) (layer F.Cu) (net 3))
 (segment (start 91.44 57.785) (end 92.71 57.785) (width 0.75) (layer F.Cu) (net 3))
 (segment (start 90.805 57.15) (end 91.44 57.785) (width 0.75) (layer F.Cu) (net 3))
 (segment (start 88.265 55.245) (end 88.265 57.785) (width 0.75) (layer F.Cu) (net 4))
 (segment (start 93.98 59.055) (end 96.52 56.515) (width 0.75) (layer F.Cu) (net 4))
 (segment (start 89.535 59.055) (end 93.98 59.055) (width 0.75) (layer F.Cu) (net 4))
 (segment (start 88.265 57.785) (end 89.535 59.055) (width 0.75) (layer F.Cu) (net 4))
 (segment (start 96.52 56.515) (end 96.52 56.41) (width 0.75) (layer F.Cu) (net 4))
 (segment (start 96.52 64.03) (end 98.53 64.03) (width 1) (layer F.Cu) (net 5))
 (segment (start 100.33 58.42) (end 101.6 58.42) (width 1) (layer F.Cu) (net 5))
 (segment (start 99.187 59.563) (end 100.33 58.42) (width 1) (layer F.Cu) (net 5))
 (segment (start 99.187 63.373) (end 99.187 59.563) (width 1) (layer F.Cu) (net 5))
 (segment (start 98.53 64.03) (end 99.187 63.373) (width 1) (layer F.Cu) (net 5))
 (segment (start 96.288 64.262) (end 93.091 64.262) (width 0.75) (layer F.Cu) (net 5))
 (segment (start 88.265 63.5) (end 89.027 64.262) (width 0.75) (layer F.Cu) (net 5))
 (segment (start 89.027 64.262) (end 93.091 64.262) (width 0.75) (layer F.Cu) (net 5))
 (segment (start 88.265 63.5) (end 88.265 61.595) (width 0.75) (layer F.Cu) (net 5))
 (segment (start 96.288 64.262) (end 96.52 64.03) (width 0.75) (layer F.Cu) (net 5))
 (segment (start 96.625 64.135) (end 96.52 64.03) (width 0.75) (layer F.Cu) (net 5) (status 30))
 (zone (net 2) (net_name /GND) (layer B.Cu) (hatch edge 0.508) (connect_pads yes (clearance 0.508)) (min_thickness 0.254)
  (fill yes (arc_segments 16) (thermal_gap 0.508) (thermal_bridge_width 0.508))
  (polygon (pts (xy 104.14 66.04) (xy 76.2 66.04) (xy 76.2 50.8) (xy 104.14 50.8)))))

